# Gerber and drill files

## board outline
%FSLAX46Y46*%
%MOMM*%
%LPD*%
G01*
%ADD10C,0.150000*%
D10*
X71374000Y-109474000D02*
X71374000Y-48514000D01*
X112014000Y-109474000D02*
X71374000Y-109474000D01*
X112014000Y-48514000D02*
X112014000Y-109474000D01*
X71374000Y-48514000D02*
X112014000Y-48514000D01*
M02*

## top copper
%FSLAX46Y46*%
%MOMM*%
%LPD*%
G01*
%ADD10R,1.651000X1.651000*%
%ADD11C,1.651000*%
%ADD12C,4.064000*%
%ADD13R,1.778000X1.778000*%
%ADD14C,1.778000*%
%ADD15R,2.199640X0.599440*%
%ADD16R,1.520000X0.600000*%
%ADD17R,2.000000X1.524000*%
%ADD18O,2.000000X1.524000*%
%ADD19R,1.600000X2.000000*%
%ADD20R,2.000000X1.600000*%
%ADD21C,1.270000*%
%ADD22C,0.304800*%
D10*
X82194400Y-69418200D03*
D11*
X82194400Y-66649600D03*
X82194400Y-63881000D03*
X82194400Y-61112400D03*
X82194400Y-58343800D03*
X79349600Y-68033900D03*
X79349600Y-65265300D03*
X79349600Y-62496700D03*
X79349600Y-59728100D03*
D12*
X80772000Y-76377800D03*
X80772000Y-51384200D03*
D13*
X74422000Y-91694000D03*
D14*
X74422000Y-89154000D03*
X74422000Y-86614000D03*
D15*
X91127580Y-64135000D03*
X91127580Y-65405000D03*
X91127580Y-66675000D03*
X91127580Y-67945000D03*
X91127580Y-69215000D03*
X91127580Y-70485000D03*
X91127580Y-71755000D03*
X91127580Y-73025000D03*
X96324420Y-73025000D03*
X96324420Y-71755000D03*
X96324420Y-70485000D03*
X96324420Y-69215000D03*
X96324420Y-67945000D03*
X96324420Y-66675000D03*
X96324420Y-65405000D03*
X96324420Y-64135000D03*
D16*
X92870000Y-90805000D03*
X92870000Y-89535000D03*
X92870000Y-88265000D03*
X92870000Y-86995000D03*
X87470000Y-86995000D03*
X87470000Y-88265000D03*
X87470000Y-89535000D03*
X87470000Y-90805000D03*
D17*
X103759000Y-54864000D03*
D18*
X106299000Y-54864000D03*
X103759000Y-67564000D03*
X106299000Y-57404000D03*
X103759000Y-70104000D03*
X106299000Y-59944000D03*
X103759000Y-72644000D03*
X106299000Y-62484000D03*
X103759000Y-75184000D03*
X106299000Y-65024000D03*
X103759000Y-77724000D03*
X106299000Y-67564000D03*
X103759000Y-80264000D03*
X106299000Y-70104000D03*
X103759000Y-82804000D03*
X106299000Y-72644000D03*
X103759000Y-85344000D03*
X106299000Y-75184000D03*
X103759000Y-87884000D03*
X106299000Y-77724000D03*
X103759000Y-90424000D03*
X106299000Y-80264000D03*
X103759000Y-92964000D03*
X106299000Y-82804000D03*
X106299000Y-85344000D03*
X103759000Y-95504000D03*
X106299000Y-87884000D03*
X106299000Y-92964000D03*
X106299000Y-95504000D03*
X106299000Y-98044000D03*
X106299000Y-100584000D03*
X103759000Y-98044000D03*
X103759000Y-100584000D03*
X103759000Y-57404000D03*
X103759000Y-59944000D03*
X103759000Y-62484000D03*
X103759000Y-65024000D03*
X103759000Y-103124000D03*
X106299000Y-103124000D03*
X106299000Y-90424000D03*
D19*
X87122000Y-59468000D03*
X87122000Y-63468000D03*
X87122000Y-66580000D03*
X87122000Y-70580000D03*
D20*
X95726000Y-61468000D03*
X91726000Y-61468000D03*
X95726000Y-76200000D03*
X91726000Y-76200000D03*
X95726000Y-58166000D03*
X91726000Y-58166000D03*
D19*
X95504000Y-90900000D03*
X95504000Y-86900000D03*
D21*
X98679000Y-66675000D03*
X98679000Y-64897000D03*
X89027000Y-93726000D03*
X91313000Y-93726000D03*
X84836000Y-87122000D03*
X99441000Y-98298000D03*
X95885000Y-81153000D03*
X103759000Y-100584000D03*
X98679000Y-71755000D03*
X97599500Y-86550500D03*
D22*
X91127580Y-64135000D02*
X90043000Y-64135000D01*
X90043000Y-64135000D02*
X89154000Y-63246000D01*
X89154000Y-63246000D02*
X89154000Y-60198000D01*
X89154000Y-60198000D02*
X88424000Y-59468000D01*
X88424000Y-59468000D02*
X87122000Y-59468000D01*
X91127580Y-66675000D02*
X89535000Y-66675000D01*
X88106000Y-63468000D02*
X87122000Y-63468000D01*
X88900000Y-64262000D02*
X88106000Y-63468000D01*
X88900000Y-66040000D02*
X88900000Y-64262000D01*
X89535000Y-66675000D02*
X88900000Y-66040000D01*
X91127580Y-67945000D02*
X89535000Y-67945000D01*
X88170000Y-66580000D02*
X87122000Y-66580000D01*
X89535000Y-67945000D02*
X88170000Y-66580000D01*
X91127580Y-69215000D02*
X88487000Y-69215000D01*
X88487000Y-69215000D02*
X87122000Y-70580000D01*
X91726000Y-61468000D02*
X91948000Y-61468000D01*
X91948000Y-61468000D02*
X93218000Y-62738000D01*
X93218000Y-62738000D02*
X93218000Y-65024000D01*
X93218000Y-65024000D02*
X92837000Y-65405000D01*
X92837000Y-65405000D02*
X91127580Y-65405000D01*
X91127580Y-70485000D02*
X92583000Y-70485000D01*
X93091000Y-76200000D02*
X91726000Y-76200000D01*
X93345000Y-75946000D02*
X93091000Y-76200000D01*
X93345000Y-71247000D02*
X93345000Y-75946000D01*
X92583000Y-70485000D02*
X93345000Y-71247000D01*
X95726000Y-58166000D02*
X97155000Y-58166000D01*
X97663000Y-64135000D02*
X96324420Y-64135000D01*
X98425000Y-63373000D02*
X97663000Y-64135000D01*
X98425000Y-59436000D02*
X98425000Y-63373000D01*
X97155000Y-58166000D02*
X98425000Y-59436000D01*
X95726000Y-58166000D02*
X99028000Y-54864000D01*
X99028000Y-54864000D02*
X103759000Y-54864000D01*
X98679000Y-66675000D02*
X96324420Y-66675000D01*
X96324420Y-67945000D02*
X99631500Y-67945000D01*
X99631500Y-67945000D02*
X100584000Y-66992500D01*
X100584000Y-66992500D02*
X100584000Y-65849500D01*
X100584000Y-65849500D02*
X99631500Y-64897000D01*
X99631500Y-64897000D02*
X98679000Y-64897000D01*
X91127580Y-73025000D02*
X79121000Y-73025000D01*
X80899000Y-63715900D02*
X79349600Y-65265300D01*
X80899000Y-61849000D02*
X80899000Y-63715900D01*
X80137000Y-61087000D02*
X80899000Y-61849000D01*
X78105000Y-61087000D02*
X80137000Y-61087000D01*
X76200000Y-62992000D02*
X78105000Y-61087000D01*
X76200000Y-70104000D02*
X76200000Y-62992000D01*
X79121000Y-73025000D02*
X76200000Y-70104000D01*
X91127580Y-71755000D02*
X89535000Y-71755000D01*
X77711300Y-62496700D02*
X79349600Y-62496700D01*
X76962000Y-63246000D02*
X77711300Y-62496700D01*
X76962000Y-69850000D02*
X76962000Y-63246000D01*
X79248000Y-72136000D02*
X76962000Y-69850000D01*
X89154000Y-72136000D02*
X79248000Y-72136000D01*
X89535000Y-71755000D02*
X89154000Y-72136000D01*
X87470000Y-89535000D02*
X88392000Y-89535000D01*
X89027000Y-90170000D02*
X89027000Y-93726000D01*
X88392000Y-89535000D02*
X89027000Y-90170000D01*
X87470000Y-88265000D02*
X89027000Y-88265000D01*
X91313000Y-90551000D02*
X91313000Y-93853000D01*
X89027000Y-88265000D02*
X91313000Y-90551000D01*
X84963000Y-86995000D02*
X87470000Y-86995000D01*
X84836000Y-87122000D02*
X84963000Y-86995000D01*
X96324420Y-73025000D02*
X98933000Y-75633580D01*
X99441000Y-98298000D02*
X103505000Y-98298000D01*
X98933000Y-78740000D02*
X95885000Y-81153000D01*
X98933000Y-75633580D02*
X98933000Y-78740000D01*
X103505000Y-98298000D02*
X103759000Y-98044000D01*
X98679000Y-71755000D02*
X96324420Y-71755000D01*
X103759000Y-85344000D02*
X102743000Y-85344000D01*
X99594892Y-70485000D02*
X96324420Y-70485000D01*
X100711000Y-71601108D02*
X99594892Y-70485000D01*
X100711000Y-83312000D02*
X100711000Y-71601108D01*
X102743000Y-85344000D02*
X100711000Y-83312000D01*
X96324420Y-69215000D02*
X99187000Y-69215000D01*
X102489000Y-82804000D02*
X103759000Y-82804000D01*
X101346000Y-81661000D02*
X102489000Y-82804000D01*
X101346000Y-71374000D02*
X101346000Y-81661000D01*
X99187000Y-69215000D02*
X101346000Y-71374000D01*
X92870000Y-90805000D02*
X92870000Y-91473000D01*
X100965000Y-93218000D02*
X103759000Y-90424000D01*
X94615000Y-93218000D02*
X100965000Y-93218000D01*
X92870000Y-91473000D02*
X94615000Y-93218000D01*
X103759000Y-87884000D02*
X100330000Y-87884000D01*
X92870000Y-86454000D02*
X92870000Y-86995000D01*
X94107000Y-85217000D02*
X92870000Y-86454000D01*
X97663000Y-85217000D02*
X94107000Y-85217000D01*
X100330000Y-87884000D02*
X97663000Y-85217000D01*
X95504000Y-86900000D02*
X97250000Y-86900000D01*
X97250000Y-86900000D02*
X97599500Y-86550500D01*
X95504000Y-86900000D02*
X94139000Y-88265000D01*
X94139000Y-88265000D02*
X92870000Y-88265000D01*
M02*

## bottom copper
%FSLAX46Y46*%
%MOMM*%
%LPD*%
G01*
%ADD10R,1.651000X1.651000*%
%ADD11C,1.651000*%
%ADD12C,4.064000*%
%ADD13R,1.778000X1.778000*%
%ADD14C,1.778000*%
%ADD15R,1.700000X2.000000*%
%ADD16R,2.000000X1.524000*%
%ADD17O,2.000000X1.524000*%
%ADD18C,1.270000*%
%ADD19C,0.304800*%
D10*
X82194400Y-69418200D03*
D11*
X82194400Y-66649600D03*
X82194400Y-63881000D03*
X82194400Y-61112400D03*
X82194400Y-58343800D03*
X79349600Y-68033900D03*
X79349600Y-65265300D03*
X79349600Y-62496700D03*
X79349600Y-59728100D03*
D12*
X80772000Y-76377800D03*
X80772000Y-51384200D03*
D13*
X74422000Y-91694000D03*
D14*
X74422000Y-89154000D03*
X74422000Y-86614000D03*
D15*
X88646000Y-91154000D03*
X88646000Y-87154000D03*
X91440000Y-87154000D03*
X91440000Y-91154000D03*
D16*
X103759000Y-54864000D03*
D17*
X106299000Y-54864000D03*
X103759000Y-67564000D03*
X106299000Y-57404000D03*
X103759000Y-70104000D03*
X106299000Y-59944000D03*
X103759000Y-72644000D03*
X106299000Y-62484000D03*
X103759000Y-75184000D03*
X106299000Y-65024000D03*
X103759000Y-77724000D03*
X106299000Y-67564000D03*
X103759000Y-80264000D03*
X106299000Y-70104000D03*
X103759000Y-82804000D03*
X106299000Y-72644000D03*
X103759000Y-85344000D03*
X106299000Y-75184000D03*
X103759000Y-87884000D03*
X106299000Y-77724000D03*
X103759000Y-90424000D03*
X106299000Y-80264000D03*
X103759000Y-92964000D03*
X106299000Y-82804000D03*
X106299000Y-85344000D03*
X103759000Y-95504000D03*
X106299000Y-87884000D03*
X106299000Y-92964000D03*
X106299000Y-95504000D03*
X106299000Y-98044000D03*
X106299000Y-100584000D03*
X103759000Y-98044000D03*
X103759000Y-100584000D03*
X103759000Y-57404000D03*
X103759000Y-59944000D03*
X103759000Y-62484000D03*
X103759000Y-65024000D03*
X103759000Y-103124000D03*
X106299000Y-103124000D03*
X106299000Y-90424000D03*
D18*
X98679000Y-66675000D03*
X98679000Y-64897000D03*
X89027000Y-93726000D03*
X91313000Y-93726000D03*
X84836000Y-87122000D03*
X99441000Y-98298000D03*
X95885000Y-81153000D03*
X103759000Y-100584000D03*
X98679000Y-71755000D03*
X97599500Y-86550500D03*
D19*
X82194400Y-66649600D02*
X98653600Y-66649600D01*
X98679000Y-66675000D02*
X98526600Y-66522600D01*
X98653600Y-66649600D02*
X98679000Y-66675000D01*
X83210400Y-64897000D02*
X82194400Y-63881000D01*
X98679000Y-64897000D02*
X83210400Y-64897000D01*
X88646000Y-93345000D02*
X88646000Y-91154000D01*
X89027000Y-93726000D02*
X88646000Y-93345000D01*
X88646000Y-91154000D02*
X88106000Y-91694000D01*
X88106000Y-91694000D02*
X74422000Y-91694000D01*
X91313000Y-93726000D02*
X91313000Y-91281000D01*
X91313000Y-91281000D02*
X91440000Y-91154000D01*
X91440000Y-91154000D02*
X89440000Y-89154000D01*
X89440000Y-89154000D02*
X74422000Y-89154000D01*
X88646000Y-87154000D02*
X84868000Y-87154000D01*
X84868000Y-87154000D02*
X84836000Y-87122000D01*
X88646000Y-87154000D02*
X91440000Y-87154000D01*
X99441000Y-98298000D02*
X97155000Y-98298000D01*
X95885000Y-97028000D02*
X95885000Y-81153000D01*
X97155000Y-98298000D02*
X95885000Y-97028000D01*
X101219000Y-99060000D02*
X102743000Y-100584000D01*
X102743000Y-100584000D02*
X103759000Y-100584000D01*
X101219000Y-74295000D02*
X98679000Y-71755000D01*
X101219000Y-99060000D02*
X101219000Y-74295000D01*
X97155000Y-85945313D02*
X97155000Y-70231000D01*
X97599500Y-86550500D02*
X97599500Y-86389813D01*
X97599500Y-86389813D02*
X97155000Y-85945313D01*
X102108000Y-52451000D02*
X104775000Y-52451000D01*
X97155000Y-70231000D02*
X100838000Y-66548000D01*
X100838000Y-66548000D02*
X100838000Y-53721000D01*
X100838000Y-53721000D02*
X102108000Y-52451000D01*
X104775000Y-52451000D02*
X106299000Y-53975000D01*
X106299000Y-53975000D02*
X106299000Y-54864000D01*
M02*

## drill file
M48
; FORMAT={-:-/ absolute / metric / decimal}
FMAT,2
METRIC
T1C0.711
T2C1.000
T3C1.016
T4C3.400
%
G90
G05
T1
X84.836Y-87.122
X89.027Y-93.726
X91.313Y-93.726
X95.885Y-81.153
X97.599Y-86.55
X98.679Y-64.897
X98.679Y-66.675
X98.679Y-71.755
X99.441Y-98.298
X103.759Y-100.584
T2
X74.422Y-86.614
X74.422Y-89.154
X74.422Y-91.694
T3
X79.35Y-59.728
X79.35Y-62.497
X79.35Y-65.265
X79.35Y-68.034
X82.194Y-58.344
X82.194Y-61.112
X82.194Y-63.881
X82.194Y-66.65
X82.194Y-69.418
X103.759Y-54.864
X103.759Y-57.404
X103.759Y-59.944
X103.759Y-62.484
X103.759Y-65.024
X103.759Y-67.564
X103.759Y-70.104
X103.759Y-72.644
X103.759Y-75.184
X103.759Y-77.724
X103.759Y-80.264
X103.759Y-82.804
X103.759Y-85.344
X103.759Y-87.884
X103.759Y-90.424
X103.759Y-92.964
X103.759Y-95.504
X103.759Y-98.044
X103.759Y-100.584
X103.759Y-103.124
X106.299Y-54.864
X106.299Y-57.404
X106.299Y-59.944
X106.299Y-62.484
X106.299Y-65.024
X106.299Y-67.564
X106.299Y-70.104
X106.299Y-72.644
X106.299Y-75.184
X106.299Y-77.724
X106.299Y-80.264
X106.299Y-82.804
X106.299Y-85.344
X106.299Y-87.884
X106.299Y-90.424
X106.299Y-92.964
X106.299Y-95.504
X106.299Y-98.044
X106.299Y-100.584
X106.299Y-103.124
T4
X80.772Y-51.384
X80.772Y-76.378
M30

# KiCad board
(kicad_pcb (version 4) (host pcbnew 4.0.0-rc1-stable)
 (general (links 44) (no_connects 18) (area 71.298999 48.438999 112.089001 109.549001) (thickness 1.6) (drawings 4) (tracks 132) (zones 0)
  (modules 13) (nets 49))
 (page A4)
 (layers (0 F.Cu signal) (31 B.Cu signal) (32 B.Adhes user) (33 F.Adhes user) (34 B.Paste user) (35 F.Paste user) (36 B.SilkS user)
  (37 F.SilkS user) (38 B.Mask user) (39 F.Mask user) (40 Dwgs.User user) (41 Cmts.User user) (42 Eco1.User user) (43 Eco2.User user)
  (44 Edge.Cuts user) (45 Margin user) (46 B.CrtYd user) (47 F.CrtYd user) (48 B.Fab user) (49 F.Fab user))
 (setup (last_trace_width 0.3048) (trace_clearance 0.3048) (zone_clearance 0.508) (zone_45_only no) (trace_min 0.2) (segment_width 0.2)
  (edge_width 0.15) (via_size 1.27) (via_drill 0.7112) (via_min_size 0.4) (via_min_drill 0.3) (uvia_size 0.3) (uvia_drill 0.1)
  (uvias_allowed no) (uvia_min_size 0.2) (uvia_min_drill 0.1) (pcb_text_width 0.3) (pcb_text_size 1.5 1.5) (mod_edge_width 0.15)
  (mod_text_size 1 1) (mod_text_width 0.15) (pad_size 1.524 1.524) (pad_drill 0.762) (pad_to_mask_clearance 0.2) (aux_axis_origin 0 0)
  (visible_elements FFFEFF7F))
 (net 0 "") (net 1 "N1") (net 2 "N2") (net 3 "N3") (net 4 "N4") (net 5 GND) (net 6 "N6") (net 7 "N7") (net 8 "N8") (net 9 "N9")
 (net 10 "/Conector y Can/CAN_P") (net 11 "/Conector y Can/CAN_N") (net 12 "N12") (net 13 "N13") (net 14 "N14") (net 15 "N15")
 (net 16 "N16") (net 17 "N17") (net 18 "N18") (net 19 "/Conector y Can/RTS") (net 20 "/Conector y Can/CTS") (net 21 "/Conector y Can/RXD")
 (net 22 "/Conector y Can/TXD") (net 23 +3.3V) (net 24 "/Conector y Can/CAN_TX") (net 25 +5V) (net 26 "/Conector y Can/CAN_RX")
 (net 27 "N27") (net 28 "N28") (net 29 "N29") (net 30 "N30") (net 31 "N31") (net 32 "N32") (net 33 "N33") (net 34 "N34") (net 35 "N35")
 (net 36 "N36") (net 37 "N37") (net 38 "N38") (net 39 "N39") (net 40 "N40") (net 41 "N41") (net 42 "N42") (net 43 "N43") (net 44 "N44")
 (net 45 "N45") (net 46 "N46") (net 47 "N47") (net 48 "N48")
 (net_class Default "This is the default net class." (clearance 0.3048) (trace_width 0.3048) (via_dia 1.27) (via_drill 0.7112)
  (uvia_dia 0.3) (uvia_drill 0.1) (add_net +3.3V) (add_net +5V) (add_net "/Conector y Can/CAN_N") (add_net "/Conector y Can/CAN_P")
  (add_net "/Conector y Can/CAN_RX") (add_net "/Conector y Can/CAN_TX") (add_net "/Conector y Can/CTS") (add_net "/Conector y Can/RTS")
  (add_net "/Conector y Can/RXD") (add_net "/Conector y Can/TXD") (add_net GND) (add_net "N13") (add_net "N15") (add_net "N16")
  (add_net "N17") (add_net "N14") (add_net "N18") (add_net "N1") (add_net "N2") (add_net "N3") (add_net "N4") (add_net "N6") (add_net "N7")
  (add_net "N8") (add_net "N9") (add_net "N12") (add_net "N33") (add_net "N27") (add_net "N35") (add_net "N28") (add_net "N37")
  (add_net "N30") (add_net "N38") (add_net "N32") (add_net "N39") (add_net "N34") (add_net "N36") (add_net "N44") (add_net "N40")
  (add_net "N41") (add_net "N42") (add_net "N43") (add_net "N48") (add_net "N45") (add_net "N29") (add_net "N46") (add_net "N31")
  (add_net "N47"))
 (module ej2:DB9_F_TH (layer F.Cu) (at 80.772 63.881 90)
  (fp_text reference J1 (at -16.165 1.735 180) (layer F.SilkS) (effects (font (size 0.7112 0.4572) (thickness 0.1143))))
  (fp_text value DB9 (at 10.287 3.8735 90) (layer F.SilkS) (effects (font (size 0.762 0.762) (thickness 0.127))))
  (pad 1 thru_hole rect (at -5.5372 1.4224 90) (size 1.651 1.651) (drill 1.016) (layers *.Cu *.Mask) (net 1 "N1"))
  (pad 2 thru_hole circle (at -2.7686 1.4224 90) (size 1.651 1.651) (drill 1.016) (layers *.Cu *.Mask) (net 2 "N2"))
  (pad 3 thru_hole circle (at 0 1.4224 90) (size 1.651 1.651) (drill 1.016) (layers *.Cu *.Mask) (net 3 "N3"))
  (pad 4 thru_hole circle (at 2.7686 1.4224 90) (size 1.651 1.651) (drill 1.016) (layers *.Cu *.Mask) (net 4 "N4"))
  (pad 5 thru_hole circle (at 5.5372 1.4224 90) (size 1.651 1.651) (drill 1.016) (layers *.Cu *.Mask) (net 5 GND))
  (pad 6 thru_hole circle (at -4.1529 -1.4224 90) (size 1.651 1.651) (drill 1.016) (layers *.Cu *.Mask) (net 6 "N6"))
  (pad 7 thru_hole circle (at -1.3843 -1.4224 90) (size 1.651 1.651) (drill 1.016) (layers *.Cu *.Mask) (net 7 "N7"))
  (pad 8 thru_hole circle (at 1.3843 -1.4224 90) (size 1.651 1.651) (drill 1.016) (layers *.Cu *.Mask) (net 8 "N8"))
  (pad 9 thru_hole circle (at 4.1529 -1.4224 90) (size 1.651 1.651) (drill 1.016) (layers *.Cu *.Mask) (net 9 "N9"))
  (pad 10 thru_hole circle (at -12.4968 0 90) (size 4.064 4.064) (drill 3.4) (layers *.Cu *.Mask))
  (pad 11 thru_hole circle (at 12.4968 0 90) (size 4.064 4.064) (drill 3.4) (layers *.Cu *.Mask)))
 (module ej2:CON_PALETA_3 (layer F.Cu) (at 74.422 89.154 90)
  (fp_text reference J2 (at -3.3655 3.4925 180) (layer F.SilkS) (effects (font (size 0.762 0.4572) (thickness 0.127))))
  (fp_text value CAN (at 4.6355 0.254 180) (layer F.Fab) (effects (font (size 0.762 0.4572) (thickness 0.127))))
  (pad 1 thru_hole rect (at -2.54 0 90) (size 1.778 1.778) (drill 1) (layers *.Cu *.Mask) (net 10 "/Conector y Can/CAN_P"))
  (pad 2 thru_hole circle (at 0 0 90) (size 1.778 1.778) (drill 1) (layers *.Cu *.Mask) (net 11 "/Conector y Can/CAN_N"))
  (pad 3 thru_hole circle (at 2.54 0 90) (size 1.778 1.778) (drill 1) (layers *.Cu *.Mask) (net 5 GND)))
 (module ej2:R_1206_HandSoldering (layer B.Cu) (at 88.646 89.154 90)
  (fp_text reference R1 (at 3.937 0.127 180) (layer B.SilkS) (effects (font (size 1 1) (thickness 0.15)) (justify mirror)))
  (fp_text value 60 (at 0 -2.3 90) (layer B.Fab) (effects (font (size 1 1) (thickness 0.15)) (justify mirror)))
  (pad 1 smd rect (at -2 0 90) (size 2 1.7) (layers B.Cu B.Paste B.Mask) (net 10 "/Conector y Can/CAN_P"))
  (pad 2 smd rect (at 2 0 90) (size 2 1.7) (layers B.Cu B.Paste B.Mask) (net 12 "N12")))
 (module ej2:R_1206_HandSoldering (layer B.Cu) (at 91.44 89.154 270)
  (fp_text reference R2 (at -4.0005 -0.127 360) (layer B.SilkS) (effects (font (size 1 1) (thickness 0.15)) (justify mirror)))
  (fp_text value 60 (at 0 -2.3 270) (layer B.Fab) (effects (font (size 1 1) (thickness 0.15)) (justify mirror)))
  (pad 1 smd rect (at -2 0 270) (size 2 1.7) (layers B.Cu B.Paste B.Mask) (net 12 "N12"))
  (pad 2 smd rect (at 2 0 270) (size 2 1.7) (layers B.Cu B.Paste B.Mask) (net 11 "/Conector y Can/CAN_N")))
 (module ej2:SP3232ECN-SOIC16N (layer F.Cu) (at 93.726 68.58 270)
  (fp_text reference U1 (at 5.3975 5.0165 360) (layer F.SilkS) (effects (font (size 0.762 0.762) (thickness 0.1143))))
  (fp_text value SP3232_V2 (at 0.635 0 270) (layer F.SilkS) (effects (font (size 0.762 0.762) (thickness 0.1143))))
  (pad 1 smd rect (at -4.445 2.59842 270) (size 0.59944 2.19964) (layers F.Cu F.Paste F.Mask) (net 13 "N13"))
  (pad 2 smd rect (at -3.175 2.59842 270) (size 0.59944 2.19964) (layers F.Cu F.Paste F.Mask) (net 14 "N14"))
  (pad 3 smd rect (at -1.905 2.59842 270) (size 0.59944 2.19964) (layers F.Cu F.Paste F.Mask) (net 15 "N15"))
  (pad 4 smd rect (at -0.635 2.59842 270) (size 0.59944 2.19964) (layers F.Cu F.Paste F.Mask) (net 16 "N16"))
  (pad 5 smd rect (at 0.635 2.59842 270) (size 0.59944 2.19964) (layers F.Cu F.Paste F.Mask) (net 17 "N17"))
  (pad 6 smd rect (at 1.905 2.59842 270) (size 0.59944 2.19964) (layers F.Cu F.Paste F.Mask) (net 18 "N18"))
  (pad 7 smd rect (at 3.175 2.59842 270) (size 0.59944 2.19964) (layers F.Cu F.Paste F.Mask) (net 8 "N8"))
  (pad 8 smd rect (at 4.445 2.59842 270) (size 0.59944 2.19964) (layers F.Cu F.Paste F.Mask) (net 7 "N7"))
  (pad 9 smd rect (at 4.445 -2.59842 270) (size 0.59944 2.19964) (layers F.Cu F.Paste F.Mask) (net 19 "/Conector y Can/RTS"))
  (pad 10 smd rect (at 3.175 -2.59842 270) (size 0.59944 2.19964) (layers F.Cu F.Paste F.Mask) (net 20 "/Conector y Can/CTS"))
  (pad 11 smd rect (at 1.905 -2.59842 270) (size 0.59944 2.19964) (layers F.Cu F.Paste F.Mask) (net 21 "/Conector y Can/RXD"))
  (pad 12 smd rect (at 0.635 -2.59842 270) (size 0.59944 2.19964) (layers F.Cu F.Paste F.Mask) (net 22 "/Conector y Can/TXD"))
  (pad 13 smd rect (at -0.635 -2.59842 270) (size 0.59944 2.19964) (layers F.Cu F.Paste F.Mask) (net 3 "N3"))
  (pad 14 smd rect (at -1.905 -2.59842 270) (size 0.59944 2.19964) (layers F.Cu F.Paste F.Mask) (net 2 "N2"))
  (pad 15 smd rect (at -3.175 -2.59842 270) (size 0.59944 2.19964) (layers F.Cu F.Paste F.Mask) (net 5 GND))
  (pad 16 smd rect (at -4.445 -2.59842 270) (size 0.59944 2.19964) (layers F.Cu F.Paste F.Mask) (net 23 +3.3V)))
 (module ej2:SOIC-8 (layer F.Cu) (at 90.17 88.9 180)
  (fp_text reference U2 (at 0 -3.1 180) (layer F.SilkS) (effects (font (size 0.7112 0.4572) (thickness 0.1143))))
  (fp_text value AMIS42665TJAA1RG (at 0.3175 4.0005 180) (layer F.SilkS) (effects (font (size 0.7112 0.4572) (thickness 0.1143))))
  (pad 1 smd rect (at -2.7 -1.905 90) (size 0.6 1.52) (layers F.Cu F.Paste F.Mask) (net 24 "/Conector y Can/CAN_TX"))
  (pad 2 smd rect (at -2.7 -0.635 90) (size 0.6 1.52) (layers F.Cu F.Paste F.Mask) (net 5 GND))
  (pad 3 smd rect (at -2.7 0.635 90) (size 0.6 1.52) (layers F.Cu F.Paste F.Mask) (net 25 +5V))
  (pad 4 smd rect (at -2.7 1.905 90) (size 0.6 1.52) (layers F.Cu F.Paste F.Mask) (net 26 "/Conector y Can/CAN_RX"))
  (pad 5 smd rect (at 2.7 1.905 90) (size 0.6 1.52) (layers F.Cu F.Paste F.Mask) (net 12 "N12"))
  (pad 6 smd rect (at 2.7 0.635 90) (size 0.6 1.52) (layers F.Cu F.Paste F.Mask) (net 11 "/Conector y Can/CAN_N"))
  (pad 7 smd rect (at 2.7 -0.635 90) (size 0.6 1.52) (layers F.Cu F.Paste F.Mask) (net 10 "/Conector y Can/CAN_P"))
  (pad 8 smd rect (at 2.7 -1.905 90) (size 0.6 1.52) (layers F.Cu F.Paste F.Mask) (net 5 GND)))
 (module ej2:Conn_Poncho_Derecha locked (layer F.Cu) (at 103.759 54.864)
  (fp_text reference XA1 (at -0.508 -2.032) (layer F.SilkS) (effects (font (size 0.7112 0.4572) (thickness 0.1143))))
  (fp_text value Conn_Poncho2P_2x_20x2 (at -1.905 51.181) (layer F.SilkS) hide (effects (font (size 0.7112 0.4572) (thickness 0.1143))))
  (pad 1 thru_hole rect (at 0 0 270) (size 1.524 2) (drill 1.016) (layers *.Cu *.Mask) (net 23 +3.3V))
  (pad 2 thru_hole oval (at 2.54 0 270) (size 1.524 2) (drill 1.016) (layers *.Cu *.Mask) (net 25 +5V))
  (pad 11 thru_hole oval (at 0 12.7 270) (size 1.524 2) (drill 1.016) (layers *.Cu *.Mask) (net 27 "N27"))
  (pad 4 thru_hole oval (at 2.54 2.54 270) (size 1.524 2) (drill 1.016) (layers *.Cu *.Mask) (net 5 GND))
  (pad 13 thru_hole oval (at 0 15.24 270) (size 1.524 2) (drill 1.016) (layers *.Cu *.Mask) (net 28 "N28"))
  (pad 6 thru_hole oval (at 2.54 5.08 270) (size 1.524 2) (drill 1.016) (layers *.Cu *.Mask) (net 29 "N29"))
  (pad 15 thru_hole oval (at 0 17.78 270) (size 1.524 2) (drill 1.016) (layers *.Cu *.Mask) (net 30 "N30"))
  (pad 8 thru_hole oval (at 2.54 7.62 270) (size 1.524 2) (drill 1.016) (layers *.Cu *.Mask) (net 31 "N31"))
  (pad 17 thru_hole oval (at 0 20.32 270) (size 1.524 2) (drill 1.016) (layers *.Cu *.Mask) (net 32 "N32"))
  (pad 10 thru_hole oval (at 2.54 10.16 270) (size 1.524 2) (drill 1.016) (layers *.Cu *.Mask) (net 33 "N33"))
  (pad 19 thru_hole oval (at 0 22.86 270) (size 1.524 2) (drill 1.016) (layers *.Cu *.Mask) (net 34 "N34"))
  (pad 12 thru_hole oval (at 2.54 12.7 270) (size 1.524 2) (drill 1.016) (layers *.Cu *.Mask) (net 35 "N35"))
  (pad 21 thru_hole oval (at 0 25.4 270) (size 1.524 2) (drill 1.016) (layers *.Cu *.Mask) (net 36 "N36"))
  (pad 14 thru_hole oval (at 2.54 15.24 270) (size 1.524 2) (drill 1.016) (layers *.Cu *.Mask) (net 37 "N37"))
  (pad 23 thru_hole oval (at 0 27.94 270) (size 1.524 2) (drill 1.016) (layers *.Cu *.Mask) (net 22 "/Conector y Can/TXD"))
  (pad 16 thru_hole oval (at 2.54 17.78 270) (size 1.524 2) (drill 1.016) (layers *.Cu *.Mask) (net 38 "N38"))
  (pad 25 thru_hole oval (at 0 30.48 270) (size 1.524 2) (drill 1.016) (layers *.Cu *.Mask) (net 21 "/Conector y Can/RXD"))
  (pad 18 thru_hole oval (at 2.54 20.32 270) (size 1.524 2) (drill 1.016) (layers *.Cu *.Mask) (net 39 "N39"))
  (pad 27 thru_hole oval (at 0 33.02 270) (size 1.524 2) (drill 1.016) (layers *.Cu *.Mask) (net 26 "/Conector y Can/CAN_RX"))
  (pad 20 thru_hole oval (at 2.54 22.86 270) (size 1.524 2) (drill 1.016) (layers *.Cu *.Mask) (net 5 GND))
  (pad 29 thru_hole oval (at 0 35.56 270) (size 1.524 2) (drill 1.016) (layers *.Cu *.Mask) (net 24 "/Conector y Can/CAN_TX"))
  (pad 22 thru_hole oval (at 2.54 25.4 270) (size 1.524 2) (drill 1.016) (layers *.Cu *.Mask) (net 5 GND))
  (pad 31 thru_hole oval (at 0 38.1 270) (size 1.524 2) (drill 1.016) (layers *.Cu *.Mask) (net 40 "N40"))
  (pad 24 thru_hole oval (at 2.54 27.94 270) (size 1.524 2) (drill 1.016) (layers *.Cu *.Mask) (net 5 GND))
  (pad 26 thru_hole oval (at 2.54 30.48 270) (size 1.524 2) (drill 1.016) (layers *.Cu *.Mask) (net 5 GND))
  (pad 33 thru_hole oval (at 0 40.64 270) (size 1.524 2) (drill 1.016) (layers *.Cu *.Mask) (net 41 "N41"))
  (pad 28 thru_hole oval (at 2.54 33.02 270) (size 1.524 2) (drill 1.016) (layers *.Cu *.Mask) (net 5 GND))
  (pad 32 thru_hole oval (at 2.54 38.1 270) (size 1.524 2) (drill 1.016) (layers *.Cu *.Mask) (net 5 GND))
  (pad 34 thru_hole oval (at 2.54 40.64 270) (size 1.524 2) (drill 1.016) (layers *.Cu *.Mask) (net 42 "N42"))
  (pad 36 thru_hole oval (at 2.54 43.18 270) (size 1.524 2) (drill 1.016) (layers *.Cu *.Mask) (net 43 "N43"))
  (pad 38 thru_hole oval (at 2.54 45.72 270) (size 1.524 2) (drill 1.016) (layers *.Cu *.Mask) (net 5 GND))
  (pad 35 thru_hole oval (at 0 43.18 270) (size 1.524 2) (drill 1.016) (layers *.Cu *.Mask) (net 19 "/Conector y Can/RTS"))
  (pad 37 thru_hole oval (at 0 45.72 270) (size 1.524 2) (drill 1.016) (layers *.Cu *.Mask) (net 20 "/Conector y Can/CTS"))
  (pad 3 thru_hole oval (at 0 2.54 270) (size 1.524 2) (drill 1.016) (layers *.Cu *.Mask) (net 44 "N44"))
  (pad 5 thru_hole oval (at 0 5.08 270) (size 1.524 2) (drill 1.016) (layers *.Cu *.Mask) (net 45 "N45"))
  (pad 7 thru_hole oval (at 0 7.62 270) (size 1.524 2) (drill 1.016) (layers *.Cu *.Mask) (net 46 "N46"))
  (pad 9 thru_hole oval (at 0 10.16 270) (size 1.524 2) (drill 1.016) (layers *.Cu *.Mask) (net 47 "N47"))
  (pad 39 thru_hole oval (at 0 48.26 270) (size 1.524 2) (drill 1.016) (layers *.Cu *.Mask) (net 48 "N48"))
  (pad 40 thru_hole oval (at 2.54 48.26 270) (size 1.524 2) (drill 1.016) (layers *.Cu *.Mask) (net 5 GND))
  (pad 30 thru_hole oval (at 2.54 35.56 270) (size 1.524 2) (drill 1.016) (layers *.Cu *.Mask) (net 5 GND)))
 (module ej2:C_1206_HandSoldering (layer F.Cu) (at 87.122 61.468 270)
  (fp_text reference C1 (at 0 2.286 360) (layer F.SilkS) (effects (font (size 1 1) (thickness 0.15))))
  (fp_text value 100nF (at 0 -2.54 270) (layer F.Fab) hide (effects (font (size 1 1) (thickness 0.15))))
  (pad 1 smd rect (at -2 0 270) (size 2 1.6) (layers F.Cu F.Paste F.Mask) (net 13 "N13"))
  (pad 2 smd rect (at 2 0 270) (size 2 1.6) (layers F.Cu F.Paste F.Mask) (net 15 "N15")))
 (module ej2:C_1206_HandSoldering (layer F.Cu) (at 87.122 68.58 270)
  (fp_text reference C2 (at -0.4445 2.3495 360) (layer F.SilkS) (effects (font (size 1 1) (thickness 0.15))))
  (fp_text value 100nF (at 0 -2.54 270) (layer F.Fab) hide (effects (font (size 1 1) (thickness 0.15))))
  (pad 1 smd rect (at -2 0 270) (size 2 1.6) (layers F.Cu F.Paste F.Mask) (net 16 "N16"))
  (pad 2 smd rect (at 2 0 270) (size 2 1.6) (layers F.Cu F.Paste F.Mask) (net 17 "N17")))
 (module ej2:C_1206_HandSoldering (layer F.Cu) (at 93.726 61.468 180)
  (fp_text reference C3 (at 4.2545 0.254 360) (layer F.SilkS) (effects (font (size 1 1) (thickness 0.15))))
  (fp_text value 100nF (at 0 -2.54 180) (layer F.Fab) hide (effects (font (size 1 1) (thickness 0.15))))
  (pad 1 smd rect (at -2 0 180) (size 2 1.6) (layers F.Cu F.Paste F.Mask) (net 5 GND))
  (pad 2 smd rect (at 2 0 180) (size 2 1.6) (layers F.Cu F.Paste F.Mask) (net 14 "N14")))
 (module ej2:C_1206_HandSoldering (layer F.Cu) (at 93.726 76.2 180)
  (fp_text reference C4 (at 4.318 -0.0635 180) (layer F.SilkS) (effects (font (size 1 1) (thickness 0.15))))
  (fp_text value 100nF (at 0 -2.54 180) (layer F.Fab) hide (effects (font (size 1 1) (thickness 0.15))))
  (pad 1 smd rect (at -2 0 180) (size 2 1.6) (layers F.Cu F.Paste F.Mask) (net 5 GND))
  (pad 2 smd rect (at 2 0 180) (size 2 1.6) (layers F.Cu F.Paste F.Mask) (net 18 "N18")))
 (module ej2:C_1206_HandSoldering (layer F.Cu) (at 93.726 58.166 180)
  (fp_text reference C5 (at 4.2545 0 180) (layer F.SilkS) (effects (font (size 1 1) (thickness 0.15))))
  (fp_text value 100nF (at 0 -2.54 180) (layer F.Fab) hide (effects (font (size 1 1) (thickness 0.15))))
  (pad 1 smd rect (at -2 0 180) (size 2 1.6) (layers F.Cu F.Paste F.Mask) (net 23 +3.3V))
  (pad 2 smd rect (at 2 0 180) (size 2 1.6) (layers F.Cu F.Paste F.Mask) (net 5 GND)))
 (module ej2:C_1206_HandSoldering (layer F.Cu) (at 95.504 88.9 90)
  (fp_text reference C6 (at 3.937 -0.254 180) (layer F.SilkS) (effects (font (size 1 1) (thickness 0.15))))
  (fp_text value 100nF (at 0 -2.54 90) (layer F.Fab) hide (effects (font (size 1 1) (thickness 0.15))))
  (pad 1 smd rect (at -2 0 90) (size 2 1.6) (layers F.Cu F.Paste F.Mask) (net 5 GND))
  (pad 2 smd rect (at 2 0 90) (size 2 1.6) (layers F.Cu F.Paste F.Mask) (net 25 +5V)))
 (gr_line (start 71.374 109.474) (end 71.374 48.514) (angle 90) (layer Edge.Cuts) (width 0.15))
 (gr_line (start 112.014 109.474) (end 71.374 109.474) (angle 90) (layer Edge.Cuts) (width 0.15))
 (gr_line (start 112.014 48.514) (end 112.014 109.474) (angle 90) (layer Edge.Cuts) (width 0.15))
 (gr_line (start 71.374 48.514) (end 112.014 48.514) (angle 90) (layer Edge.Cuts) (width 0.15))
 (segment (start 91.12758 64.135) (end 90.043 64.135) (width 0.3048) (layer F.Cu) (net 13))
 (segment (start 90.043 64.135) (end 89.154 63.246) (width 0.3048) (layer F.Cu) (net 13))
 (segment (start 89.154 63.246) (end 89.154 60.198) (width 0.3048) (layer F.Cu) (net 13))
 (segment (start 89.154 60.198) (end 88.424 59.468) (width 0.3048) (layer F.Cu) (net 13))
 (segment (start 88.424 59.468) (end 87.122 59.468) (width 0.3048) (layer F.Cu) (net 13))
 (segment (start 91.12758 66.675) (end 89.535 66.675) (width 0.3048) (layer F.Cu) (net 15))
 (segment (start 88.106 63.468) (end 87.122 63.468) (width 0.3048) (layer F.Cu) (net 15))
 (segment (start 88.9 64.262) (end 88.106 63.468) (width 0.3048) (layer F.Cu) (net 15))
 (segment (start 88.9 66.04) (end 88.9 64.262) (width 0.3048) (layer F.Cu) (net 15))
 (segment (start 89.535 66.675) (end 88.9 66.04) (width 0.3048) (layer F.Cu) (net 15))
 (segment (start 91.12758 67.945) (end 89.535 67.945) (width 0.3048) (layer F.Cu) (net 16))
 (segment (start 88.17 66.58) (end 87.122 66.58) (width 0.3048) (layer F.Cu) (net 16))
 (segment (start 89.535 67.945) (end 88.17 66.58) (width 0.3048) (layer F.Cu) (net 16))
 (segment (start 91.12758 69.215) (end 88.487 69.215) (width 0.3048) (layer F.Cu) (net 17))
 (segment (start 88.487 69.215) (end 87.122 70.58) (width 0.3048) (layer F.Cu) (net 17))
 (segment (start 91.726 61.468) (end 91.948 61.468) (width 0.3048) (layer F.Cu) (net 14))
 (segment (start 91.948 61.468) (end 93.218 62.738) (width 0.3048) (layer F.Cu) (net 14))
 (segment (start 93.218 62.738) (end 93.218 65.024) (width 0.3048) (layer F.Cu) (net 14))
 (segment (start 93.218 65.024) (end 92.837 65.405) (width 0.3048) (layer F.Cu) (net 14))
 (segment (start 92.837 65.405) (end 91.12758 65.405) (width 0.3048) (layer F.Cu) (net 14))
 (segment (start 91.12758 70.485) (end 92.583 70.485) (width 0.3048) (layer F.Cu) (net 18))
 (segment (start 93.091 76.2) (end 91.726 76.2) (width 0.3048) (layer F.Cu) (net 18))
 (segment (start 93.345 75.946) (end 93.091 76.2) (width 0.3048) (layer F.Cu) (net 18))
 (segment (start 93.345 71.247) (end 93.345 75.946) (width 0.3048) (layer F.Cu) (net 18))
 (segment (start 92.583 70.485) (end 93.345 71.247) (width 0.3048) (layer F.Cu) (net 18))
 (segment (start 95.726 58.166) (end 97.155 58.166) (width 0.3048) (layer F.Cu) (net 23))
 (segment (start 97.663 64.135) (end 96.32442 64.135) (width 0.3048) (layer F.Cu) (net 23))
 (segment (start 98.425 63.373) (end 97.663 64.135) (width 0.3048) (layer F.Cu) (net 23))
 (segment (start 98.425 59.436) (end 98.425 63.373) (width 0.3048) (layer F.Cu) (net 23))
 (segment (start 97.155 58.166) (end 98.425 59.436) (width 0.3048) (layer F.Cu) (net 23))
 (segment (start 95.726 58.166) (end 99.028 54.864) (width 0.3048) (layer F.Cu) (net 23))
 (segment (start 99.028 54.864) (end 103.759 54.864) (width 0.3048) (layer F.Cu) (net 23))
 (segment (start 98.679 66.675) (end 96.32442 66.675) (width 0.3048) (layer F.Cu) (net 2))
 (segment (start 82.1944 66.6496) (end 98.6536 66.6496) (width 0.3048) (layer B.Cu) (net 2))
 (via (at 98.679 66.675) (size 1.27) (drill 0.7112) (layers F.Cu B.Cu) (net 2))
 (segment (start 98.679 66.675) (end 98.5266 66.5226) (width 0.3048) (layer B.Cu) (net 2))
 (segment (start 98.6536 66.6496) (end 98.679 66.675) (width 0.3048) (layer B.Cu) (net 2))
 (segment (start 96.32442 67.945) (end 99.6315 67.945) (width 0.3048) (layer F.Cu) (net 3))
 (segment (start 99.6315 67.945) (end 100.584 66.9925) (width 0.3048) (layer F.Cu) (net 3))
 (segment (start 100.584 66.9925) (end 100.584 65.8495) (width 0.3048) (layer F.Cu) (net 3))
 (segment (start 100.584 65.8495) (end 99.6315 64.897) (width 0.3048) (layer F.Cu) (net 3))
 (segment (start 99.6315 64.897) (end 98.679 64.897) (width 0.3048) (layer F.Cu) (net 3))
 (segment (start 83.2104 64.897) (end 82.1944 63.881) (width 0.3048) (layer B.Cu) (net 3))
 (segment (start 98.679 64.897) (end 83.2104 64.897) (width 0.3048) (layer B.Cu) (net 3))
 (via (at 98.679 64.897) (size 1.27) (drill 0.7112) (layers F.Cu B.Cu) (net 3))
 (segment (start 91.12758 73.025) (end 79.121 73.025) (width 0.3048) (layer F.Cu) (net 7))
 (segment (start 80.899 63.7159) (end 79.3496 65.2653) (width 0.3048) (layer F.Cu) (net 7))
 (segment (start 80.899 61.849) (end 80.899 63.7159) (width 0.3048) (layer F.Cu) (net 7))
 (segment (start 80.137 61.087) (end 80.899 61.849) (width 0.3048) (layer F.Cu) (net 7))
 (segment (start 78.105 61.087) (end 80.137 61.087) (width 0.3048) (layer F.Cu) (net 7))
 (segment (start 76.2 62.992) (end 78.105 61.087) (width 0.3048) (layer F.Cu) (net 7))
 (segment (start 76.2 70.104) (end 76.2 62.992) (width 0.3048) (layer F.Cu) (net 7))
 (segment (start 79.121 73.025) (end 76.2 70.104) (width 0.3048) (layer F.Cu) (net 7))
 (segment (start 91.12758 71.755) (end 89.535 71.755) (width 0.3048) (layer F.Cu) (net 8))
 (segment (start 77.7113 62.4967) (end 79.3496 62.4967) (width 0.3048) (layer F.Cu) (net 8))
 (segment (start 76.962 63.246) (end 77.7113 62.4967) (width 0.3048) (layer F.Cu) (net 8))
 (segment (start 76.962 69.85) (end 76.962 63.246) (width 0.3048) (layer F.Cu) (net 8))
 (segment (start 79.248 72.136) (end 76.962 69.85) (width 0.3048) (layer F.Cu) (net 8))
 (segment (start 89.154 72.136) (end 79.248 72.136) (width 0.3048) (layer F.Cu) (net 8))
 (segment (start 89.535 71.755) (end 89.154 72.136) (width 0.3048) (layer F.Cu) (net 8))
 (segment (start 87.47 89.535) (end 88.392 89.535) (width 0.3048) (layer F.Cu) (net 10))
 (segment (start 88.646 93.345) (end 88.646 91.154) (width 0.3048) (layer B.Cu) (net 10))
 (segment (start 89.027 93.726) (end 88.646 93.345) (width 0.3048) (layer B.Cu) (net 10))
 (via (at 89.027 93.726) (size 1.27) (drill 0.7112) (layers F.Cu B.Cu) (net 10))
 (segment (start 89.027 90.17) (end 89.027 93.726) (width 0.3048) (layer F.Cu) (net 10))
 (segment (start 88.392 89.535) (end 89.027 90.17) (width 0.3048) (layer F.Cu) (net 10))
 (segment (start 88.646 91.154) (end 88.106 91.694) (width 0.3048) (layer B.Cu) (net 10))
 (segment (start 88.106 91.694) (end 74.422 91.694) (width 0.3048) (layer B.Cu) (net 10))
 (segment (start 91.313 93.726) (end 91.313 91.281) (width 0.3048) (layer B.Cu) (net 11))
 (segment (start 91.313 91.281) (end 91.44 91.154) (width 0.3048) (layer B.Cu) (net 11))
 (segment (start 87.47 88.265) (end 89.027 88.265) (width 0.3048) (layer F.Cu) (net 11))
 (via (at 91.313 93.726) (size 1.27) (drill 0.7112) (layers F.Cu B.Cu) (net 11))
 (segment (start 91.313 90.551) (end 91.313 93.853) (width 0.3048) (layer F.Cu) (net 11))
 (segment (start 89.027 88.265) (end 91.313 90.551) (width 0.3048) (layer F.Cu) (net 11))
 (segment (start 91.44 91.154) (end 89.44 89.154) (width 0.3048) (layer B.Cu) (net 11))
 (segment (start 89.44 89.154) (end 74.422 89.154) (width 0.3048) (layer B.Cu) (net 11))
 (segment (start 88.646 87.154) (end 84.868 87.154) (width 0.3048) (layer B.Cu) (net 12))
 (segment (start 84.963 86.995) (end 87.47 86.995) (width 0.3048) (layer F.Cu) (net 12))
 (segment (start 84.836 87.122) (end 84.963 86.995) (width 0.3048) (layer F.Cu) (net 12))
 (via (at 84.836 87.122) (size 1.27) (drill 0.7112) (layers F.Cu B.Cu) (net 12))
 (segment (start 84.868 87.154) (end 84.836 87.122) (width 0.3048) (layer B.Cu) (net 12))
 (segment (start 88.646 87.154) (end 91.44 87.154) (width 0.3048) (layer B.Cu) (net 12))
 (segment (start 99.441 98.298) (end 97.155 98.298) (width 0.3048) (layer B.Cu) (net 19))
 (segment (start 95.885 97.028) (end 95.885 81.153) (width 0.3048) (layer B.Cu) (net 19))
 (segment (start 97.155 98.298) (end 95.885 97.028) (width 0.3048) (layer B.Cu) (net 19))
 (segment (start 96.32442 73.025) (end 98.933 75.63358) (width 0.3048) (layer F.Cu) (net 19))
 (segment (start 99.441 98.298) (end 103.505 98.298) (width 0.3048) (layer F.Cu) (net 19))
 (via (at 99.441 98.298) (size 1.27) (drill 0.7112) (layers F.Cu B.Cu) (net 19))
 (via (at 95.885 81.153) (size 1.27) (drill 0.7112) (layers F.Cu B.Cu) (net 19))
 (segment (start 98.933 78.74) (end 95.885 81.153) (width 0.3048) (layer F.Cu) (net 19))
 (segment (start 98.933 75.63358) (end 98.933 78.74) (width 0.3048) (layer F.Cu) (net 19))
 (segment (start 103.505 98.298) (end 103.759 98.044) (width 0.3048) (layer F.Cu) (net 19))
 (segment (start 101.219 99.06) (end 102.743 100.584) (width 0.3048) (layer B.Cu) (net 20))
 (segment (start 102.743 100.584) (end 103.759 100.584) (width 0.3048) (layer B.Cu) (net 20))
 (via (at 103.759 100.584) (size 1.27) (drill 0.7112) (layers F.Cu B.Cu) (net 20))
 (segment (start 98.679 71.755) (end 96.32442 71.755) (width 0.3048) (layer F.Cu) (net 20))
 (via (at 98.679 71.755) (size 1.27) (drill 0.7112) (layers F.Cu B.Cu) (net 20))
 (segment (start 101.219 74.295) (end 98.679 71.755) (width 0.3048) (layer B.Cu) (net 20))
 (segment (start 101.219 99.06) (end 101.219 74.295) (width 0.3048) (layer B.Cu) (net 20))
 (segment (start 103.759 85.344) (end 102.743 85.344) (width 0.3048) (layer F.Cu) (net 21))
 (segment (start 99.594892 70.485) (end 96.32442 70.485) (width 0.3048) (layer F.Cu) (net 21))
 (segment (start 100.711 71.601108) (end 99.594892 70.485) (width 0.3048) (layer F.Cu) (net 21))
 (segment (start 100.711 83.312) (end 100.711 71.601108) (width 0.3048) (layer F.Cu) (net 21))
 (segment (start 102.743 85.344) (end 100.711 83.312) (width 0.3048) (layer F.Cu) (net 21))
 (segment (start 96.32442 69.215) (end 99.187 69.215) (width 0.3048) (layer F.Cu) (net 22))
 (segment (start 102.489 82.804) (end 103.759 82.804) (width 0.3048) (layer F.Cu) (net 22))
 (segment (start 101.346 81.661) (end 102.489 82.804) (width 0.3048) (layer F.Cu) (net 22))
 (segment (start 101.346 71.374) (end 101.346 81.661) (width 0.3048) (layer F.Cu) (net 22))
 (segment (start 99.187 69.215) (end 101.346 71.374) (width 0.3048) (layer F.Cu) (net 22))
 (segment (start 92.87 90.805) (end 92.87 91.473) (width 0.3048) (layer F.Cu) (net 24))
 (segment (start 100.965 93.218) (end 103.759 90.424) (width 0.3048) (layer F.Cu) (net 24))
 (segment (start 94.615 93.218) (end 100.965 93.218) (width 0.3048) (layer F.Cu) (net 24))
 (segment (start 92.87 91.473) (end 94.615 93.218) (width 0.3048) (layer F.Cu) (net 24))
 (segment (start 103.759 87.884) (end 100.33 87.884) (width 0.3048) (layer F.Cu) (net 26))
 (segment (start 92.87 86.454) (end 92.87 86.995) (width 0.3048) (layer F.Cu) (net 26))
 (segment (start 94.107 85.217) (end 92.87 86.454) (width 0.3048) (layer F.Cu) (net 26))
 (segment (start 97.663 85.217) (end 94.107 85.217) (width 0.3048) (layer F.Cu) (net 26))
 (segment (start 100.33 87.884) (end 97.663 85.217) (width 0.3048) (layer F.Cu) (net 26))
 (segment (start 97.155 85.945313) (end 97.155 70.231) (width 0.3048) (layer B.Cu) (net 25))
 (segment (start 97.5995 86.5505) (end 97.5995 86.389813) (width 0.3048) (layer B.Cu) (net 25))
 (segment (start 97.5995 86.389813) (end 97.155 85.945313) (width 0.3048) (layer B.Cu) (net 25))
 (segment (start 95.504 86.9) (end 97.25 86.9) (width 0.3048) (layer F.Cu) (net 25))
 (segment (start 97.25 86.9) (end 97.5995 86.5505) (width 0.3048) (layer F.Cu) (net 25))
 (segment (start 102.108 52.451) (end 104.775 52.451) (width 0.3048) (layer B.Cu) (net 25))
 (segment (start 97.155 70.231) (end 100.838 66.548) (width 0.3048) (layer B.Cu) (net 25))
 (segment (start 100.838 66.548) (end 100.838 53.721) (width 0.3048) (layer B.Cu) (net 25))
 (segment (start 100.838 53.721) (end 102.108 52.451) (width 0.3048) (layer B.Cu) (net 25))
 (segment (start 104.775 52.451) (end 106.299 53.975) (width 0.3048) (layer B.Cu) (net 25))
 (segment (start 106.299 53.975) (end 106.299 54.864) (width 0.3048) (layer B.Cu) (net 25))
 (via (at 97.5995 86.5505) (size 1.27) (drill 0.7112) (layers F.Cu B.Cu) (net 25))
 (segment (start 95.504 86.9) (end 94.139 88.265) (width 0.3048) (layer F.Cu) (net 25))
 (segment (start 94.139 88.265) (end 92.87 88.265) (width 0.3048) (layer F.Cu) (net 25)))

